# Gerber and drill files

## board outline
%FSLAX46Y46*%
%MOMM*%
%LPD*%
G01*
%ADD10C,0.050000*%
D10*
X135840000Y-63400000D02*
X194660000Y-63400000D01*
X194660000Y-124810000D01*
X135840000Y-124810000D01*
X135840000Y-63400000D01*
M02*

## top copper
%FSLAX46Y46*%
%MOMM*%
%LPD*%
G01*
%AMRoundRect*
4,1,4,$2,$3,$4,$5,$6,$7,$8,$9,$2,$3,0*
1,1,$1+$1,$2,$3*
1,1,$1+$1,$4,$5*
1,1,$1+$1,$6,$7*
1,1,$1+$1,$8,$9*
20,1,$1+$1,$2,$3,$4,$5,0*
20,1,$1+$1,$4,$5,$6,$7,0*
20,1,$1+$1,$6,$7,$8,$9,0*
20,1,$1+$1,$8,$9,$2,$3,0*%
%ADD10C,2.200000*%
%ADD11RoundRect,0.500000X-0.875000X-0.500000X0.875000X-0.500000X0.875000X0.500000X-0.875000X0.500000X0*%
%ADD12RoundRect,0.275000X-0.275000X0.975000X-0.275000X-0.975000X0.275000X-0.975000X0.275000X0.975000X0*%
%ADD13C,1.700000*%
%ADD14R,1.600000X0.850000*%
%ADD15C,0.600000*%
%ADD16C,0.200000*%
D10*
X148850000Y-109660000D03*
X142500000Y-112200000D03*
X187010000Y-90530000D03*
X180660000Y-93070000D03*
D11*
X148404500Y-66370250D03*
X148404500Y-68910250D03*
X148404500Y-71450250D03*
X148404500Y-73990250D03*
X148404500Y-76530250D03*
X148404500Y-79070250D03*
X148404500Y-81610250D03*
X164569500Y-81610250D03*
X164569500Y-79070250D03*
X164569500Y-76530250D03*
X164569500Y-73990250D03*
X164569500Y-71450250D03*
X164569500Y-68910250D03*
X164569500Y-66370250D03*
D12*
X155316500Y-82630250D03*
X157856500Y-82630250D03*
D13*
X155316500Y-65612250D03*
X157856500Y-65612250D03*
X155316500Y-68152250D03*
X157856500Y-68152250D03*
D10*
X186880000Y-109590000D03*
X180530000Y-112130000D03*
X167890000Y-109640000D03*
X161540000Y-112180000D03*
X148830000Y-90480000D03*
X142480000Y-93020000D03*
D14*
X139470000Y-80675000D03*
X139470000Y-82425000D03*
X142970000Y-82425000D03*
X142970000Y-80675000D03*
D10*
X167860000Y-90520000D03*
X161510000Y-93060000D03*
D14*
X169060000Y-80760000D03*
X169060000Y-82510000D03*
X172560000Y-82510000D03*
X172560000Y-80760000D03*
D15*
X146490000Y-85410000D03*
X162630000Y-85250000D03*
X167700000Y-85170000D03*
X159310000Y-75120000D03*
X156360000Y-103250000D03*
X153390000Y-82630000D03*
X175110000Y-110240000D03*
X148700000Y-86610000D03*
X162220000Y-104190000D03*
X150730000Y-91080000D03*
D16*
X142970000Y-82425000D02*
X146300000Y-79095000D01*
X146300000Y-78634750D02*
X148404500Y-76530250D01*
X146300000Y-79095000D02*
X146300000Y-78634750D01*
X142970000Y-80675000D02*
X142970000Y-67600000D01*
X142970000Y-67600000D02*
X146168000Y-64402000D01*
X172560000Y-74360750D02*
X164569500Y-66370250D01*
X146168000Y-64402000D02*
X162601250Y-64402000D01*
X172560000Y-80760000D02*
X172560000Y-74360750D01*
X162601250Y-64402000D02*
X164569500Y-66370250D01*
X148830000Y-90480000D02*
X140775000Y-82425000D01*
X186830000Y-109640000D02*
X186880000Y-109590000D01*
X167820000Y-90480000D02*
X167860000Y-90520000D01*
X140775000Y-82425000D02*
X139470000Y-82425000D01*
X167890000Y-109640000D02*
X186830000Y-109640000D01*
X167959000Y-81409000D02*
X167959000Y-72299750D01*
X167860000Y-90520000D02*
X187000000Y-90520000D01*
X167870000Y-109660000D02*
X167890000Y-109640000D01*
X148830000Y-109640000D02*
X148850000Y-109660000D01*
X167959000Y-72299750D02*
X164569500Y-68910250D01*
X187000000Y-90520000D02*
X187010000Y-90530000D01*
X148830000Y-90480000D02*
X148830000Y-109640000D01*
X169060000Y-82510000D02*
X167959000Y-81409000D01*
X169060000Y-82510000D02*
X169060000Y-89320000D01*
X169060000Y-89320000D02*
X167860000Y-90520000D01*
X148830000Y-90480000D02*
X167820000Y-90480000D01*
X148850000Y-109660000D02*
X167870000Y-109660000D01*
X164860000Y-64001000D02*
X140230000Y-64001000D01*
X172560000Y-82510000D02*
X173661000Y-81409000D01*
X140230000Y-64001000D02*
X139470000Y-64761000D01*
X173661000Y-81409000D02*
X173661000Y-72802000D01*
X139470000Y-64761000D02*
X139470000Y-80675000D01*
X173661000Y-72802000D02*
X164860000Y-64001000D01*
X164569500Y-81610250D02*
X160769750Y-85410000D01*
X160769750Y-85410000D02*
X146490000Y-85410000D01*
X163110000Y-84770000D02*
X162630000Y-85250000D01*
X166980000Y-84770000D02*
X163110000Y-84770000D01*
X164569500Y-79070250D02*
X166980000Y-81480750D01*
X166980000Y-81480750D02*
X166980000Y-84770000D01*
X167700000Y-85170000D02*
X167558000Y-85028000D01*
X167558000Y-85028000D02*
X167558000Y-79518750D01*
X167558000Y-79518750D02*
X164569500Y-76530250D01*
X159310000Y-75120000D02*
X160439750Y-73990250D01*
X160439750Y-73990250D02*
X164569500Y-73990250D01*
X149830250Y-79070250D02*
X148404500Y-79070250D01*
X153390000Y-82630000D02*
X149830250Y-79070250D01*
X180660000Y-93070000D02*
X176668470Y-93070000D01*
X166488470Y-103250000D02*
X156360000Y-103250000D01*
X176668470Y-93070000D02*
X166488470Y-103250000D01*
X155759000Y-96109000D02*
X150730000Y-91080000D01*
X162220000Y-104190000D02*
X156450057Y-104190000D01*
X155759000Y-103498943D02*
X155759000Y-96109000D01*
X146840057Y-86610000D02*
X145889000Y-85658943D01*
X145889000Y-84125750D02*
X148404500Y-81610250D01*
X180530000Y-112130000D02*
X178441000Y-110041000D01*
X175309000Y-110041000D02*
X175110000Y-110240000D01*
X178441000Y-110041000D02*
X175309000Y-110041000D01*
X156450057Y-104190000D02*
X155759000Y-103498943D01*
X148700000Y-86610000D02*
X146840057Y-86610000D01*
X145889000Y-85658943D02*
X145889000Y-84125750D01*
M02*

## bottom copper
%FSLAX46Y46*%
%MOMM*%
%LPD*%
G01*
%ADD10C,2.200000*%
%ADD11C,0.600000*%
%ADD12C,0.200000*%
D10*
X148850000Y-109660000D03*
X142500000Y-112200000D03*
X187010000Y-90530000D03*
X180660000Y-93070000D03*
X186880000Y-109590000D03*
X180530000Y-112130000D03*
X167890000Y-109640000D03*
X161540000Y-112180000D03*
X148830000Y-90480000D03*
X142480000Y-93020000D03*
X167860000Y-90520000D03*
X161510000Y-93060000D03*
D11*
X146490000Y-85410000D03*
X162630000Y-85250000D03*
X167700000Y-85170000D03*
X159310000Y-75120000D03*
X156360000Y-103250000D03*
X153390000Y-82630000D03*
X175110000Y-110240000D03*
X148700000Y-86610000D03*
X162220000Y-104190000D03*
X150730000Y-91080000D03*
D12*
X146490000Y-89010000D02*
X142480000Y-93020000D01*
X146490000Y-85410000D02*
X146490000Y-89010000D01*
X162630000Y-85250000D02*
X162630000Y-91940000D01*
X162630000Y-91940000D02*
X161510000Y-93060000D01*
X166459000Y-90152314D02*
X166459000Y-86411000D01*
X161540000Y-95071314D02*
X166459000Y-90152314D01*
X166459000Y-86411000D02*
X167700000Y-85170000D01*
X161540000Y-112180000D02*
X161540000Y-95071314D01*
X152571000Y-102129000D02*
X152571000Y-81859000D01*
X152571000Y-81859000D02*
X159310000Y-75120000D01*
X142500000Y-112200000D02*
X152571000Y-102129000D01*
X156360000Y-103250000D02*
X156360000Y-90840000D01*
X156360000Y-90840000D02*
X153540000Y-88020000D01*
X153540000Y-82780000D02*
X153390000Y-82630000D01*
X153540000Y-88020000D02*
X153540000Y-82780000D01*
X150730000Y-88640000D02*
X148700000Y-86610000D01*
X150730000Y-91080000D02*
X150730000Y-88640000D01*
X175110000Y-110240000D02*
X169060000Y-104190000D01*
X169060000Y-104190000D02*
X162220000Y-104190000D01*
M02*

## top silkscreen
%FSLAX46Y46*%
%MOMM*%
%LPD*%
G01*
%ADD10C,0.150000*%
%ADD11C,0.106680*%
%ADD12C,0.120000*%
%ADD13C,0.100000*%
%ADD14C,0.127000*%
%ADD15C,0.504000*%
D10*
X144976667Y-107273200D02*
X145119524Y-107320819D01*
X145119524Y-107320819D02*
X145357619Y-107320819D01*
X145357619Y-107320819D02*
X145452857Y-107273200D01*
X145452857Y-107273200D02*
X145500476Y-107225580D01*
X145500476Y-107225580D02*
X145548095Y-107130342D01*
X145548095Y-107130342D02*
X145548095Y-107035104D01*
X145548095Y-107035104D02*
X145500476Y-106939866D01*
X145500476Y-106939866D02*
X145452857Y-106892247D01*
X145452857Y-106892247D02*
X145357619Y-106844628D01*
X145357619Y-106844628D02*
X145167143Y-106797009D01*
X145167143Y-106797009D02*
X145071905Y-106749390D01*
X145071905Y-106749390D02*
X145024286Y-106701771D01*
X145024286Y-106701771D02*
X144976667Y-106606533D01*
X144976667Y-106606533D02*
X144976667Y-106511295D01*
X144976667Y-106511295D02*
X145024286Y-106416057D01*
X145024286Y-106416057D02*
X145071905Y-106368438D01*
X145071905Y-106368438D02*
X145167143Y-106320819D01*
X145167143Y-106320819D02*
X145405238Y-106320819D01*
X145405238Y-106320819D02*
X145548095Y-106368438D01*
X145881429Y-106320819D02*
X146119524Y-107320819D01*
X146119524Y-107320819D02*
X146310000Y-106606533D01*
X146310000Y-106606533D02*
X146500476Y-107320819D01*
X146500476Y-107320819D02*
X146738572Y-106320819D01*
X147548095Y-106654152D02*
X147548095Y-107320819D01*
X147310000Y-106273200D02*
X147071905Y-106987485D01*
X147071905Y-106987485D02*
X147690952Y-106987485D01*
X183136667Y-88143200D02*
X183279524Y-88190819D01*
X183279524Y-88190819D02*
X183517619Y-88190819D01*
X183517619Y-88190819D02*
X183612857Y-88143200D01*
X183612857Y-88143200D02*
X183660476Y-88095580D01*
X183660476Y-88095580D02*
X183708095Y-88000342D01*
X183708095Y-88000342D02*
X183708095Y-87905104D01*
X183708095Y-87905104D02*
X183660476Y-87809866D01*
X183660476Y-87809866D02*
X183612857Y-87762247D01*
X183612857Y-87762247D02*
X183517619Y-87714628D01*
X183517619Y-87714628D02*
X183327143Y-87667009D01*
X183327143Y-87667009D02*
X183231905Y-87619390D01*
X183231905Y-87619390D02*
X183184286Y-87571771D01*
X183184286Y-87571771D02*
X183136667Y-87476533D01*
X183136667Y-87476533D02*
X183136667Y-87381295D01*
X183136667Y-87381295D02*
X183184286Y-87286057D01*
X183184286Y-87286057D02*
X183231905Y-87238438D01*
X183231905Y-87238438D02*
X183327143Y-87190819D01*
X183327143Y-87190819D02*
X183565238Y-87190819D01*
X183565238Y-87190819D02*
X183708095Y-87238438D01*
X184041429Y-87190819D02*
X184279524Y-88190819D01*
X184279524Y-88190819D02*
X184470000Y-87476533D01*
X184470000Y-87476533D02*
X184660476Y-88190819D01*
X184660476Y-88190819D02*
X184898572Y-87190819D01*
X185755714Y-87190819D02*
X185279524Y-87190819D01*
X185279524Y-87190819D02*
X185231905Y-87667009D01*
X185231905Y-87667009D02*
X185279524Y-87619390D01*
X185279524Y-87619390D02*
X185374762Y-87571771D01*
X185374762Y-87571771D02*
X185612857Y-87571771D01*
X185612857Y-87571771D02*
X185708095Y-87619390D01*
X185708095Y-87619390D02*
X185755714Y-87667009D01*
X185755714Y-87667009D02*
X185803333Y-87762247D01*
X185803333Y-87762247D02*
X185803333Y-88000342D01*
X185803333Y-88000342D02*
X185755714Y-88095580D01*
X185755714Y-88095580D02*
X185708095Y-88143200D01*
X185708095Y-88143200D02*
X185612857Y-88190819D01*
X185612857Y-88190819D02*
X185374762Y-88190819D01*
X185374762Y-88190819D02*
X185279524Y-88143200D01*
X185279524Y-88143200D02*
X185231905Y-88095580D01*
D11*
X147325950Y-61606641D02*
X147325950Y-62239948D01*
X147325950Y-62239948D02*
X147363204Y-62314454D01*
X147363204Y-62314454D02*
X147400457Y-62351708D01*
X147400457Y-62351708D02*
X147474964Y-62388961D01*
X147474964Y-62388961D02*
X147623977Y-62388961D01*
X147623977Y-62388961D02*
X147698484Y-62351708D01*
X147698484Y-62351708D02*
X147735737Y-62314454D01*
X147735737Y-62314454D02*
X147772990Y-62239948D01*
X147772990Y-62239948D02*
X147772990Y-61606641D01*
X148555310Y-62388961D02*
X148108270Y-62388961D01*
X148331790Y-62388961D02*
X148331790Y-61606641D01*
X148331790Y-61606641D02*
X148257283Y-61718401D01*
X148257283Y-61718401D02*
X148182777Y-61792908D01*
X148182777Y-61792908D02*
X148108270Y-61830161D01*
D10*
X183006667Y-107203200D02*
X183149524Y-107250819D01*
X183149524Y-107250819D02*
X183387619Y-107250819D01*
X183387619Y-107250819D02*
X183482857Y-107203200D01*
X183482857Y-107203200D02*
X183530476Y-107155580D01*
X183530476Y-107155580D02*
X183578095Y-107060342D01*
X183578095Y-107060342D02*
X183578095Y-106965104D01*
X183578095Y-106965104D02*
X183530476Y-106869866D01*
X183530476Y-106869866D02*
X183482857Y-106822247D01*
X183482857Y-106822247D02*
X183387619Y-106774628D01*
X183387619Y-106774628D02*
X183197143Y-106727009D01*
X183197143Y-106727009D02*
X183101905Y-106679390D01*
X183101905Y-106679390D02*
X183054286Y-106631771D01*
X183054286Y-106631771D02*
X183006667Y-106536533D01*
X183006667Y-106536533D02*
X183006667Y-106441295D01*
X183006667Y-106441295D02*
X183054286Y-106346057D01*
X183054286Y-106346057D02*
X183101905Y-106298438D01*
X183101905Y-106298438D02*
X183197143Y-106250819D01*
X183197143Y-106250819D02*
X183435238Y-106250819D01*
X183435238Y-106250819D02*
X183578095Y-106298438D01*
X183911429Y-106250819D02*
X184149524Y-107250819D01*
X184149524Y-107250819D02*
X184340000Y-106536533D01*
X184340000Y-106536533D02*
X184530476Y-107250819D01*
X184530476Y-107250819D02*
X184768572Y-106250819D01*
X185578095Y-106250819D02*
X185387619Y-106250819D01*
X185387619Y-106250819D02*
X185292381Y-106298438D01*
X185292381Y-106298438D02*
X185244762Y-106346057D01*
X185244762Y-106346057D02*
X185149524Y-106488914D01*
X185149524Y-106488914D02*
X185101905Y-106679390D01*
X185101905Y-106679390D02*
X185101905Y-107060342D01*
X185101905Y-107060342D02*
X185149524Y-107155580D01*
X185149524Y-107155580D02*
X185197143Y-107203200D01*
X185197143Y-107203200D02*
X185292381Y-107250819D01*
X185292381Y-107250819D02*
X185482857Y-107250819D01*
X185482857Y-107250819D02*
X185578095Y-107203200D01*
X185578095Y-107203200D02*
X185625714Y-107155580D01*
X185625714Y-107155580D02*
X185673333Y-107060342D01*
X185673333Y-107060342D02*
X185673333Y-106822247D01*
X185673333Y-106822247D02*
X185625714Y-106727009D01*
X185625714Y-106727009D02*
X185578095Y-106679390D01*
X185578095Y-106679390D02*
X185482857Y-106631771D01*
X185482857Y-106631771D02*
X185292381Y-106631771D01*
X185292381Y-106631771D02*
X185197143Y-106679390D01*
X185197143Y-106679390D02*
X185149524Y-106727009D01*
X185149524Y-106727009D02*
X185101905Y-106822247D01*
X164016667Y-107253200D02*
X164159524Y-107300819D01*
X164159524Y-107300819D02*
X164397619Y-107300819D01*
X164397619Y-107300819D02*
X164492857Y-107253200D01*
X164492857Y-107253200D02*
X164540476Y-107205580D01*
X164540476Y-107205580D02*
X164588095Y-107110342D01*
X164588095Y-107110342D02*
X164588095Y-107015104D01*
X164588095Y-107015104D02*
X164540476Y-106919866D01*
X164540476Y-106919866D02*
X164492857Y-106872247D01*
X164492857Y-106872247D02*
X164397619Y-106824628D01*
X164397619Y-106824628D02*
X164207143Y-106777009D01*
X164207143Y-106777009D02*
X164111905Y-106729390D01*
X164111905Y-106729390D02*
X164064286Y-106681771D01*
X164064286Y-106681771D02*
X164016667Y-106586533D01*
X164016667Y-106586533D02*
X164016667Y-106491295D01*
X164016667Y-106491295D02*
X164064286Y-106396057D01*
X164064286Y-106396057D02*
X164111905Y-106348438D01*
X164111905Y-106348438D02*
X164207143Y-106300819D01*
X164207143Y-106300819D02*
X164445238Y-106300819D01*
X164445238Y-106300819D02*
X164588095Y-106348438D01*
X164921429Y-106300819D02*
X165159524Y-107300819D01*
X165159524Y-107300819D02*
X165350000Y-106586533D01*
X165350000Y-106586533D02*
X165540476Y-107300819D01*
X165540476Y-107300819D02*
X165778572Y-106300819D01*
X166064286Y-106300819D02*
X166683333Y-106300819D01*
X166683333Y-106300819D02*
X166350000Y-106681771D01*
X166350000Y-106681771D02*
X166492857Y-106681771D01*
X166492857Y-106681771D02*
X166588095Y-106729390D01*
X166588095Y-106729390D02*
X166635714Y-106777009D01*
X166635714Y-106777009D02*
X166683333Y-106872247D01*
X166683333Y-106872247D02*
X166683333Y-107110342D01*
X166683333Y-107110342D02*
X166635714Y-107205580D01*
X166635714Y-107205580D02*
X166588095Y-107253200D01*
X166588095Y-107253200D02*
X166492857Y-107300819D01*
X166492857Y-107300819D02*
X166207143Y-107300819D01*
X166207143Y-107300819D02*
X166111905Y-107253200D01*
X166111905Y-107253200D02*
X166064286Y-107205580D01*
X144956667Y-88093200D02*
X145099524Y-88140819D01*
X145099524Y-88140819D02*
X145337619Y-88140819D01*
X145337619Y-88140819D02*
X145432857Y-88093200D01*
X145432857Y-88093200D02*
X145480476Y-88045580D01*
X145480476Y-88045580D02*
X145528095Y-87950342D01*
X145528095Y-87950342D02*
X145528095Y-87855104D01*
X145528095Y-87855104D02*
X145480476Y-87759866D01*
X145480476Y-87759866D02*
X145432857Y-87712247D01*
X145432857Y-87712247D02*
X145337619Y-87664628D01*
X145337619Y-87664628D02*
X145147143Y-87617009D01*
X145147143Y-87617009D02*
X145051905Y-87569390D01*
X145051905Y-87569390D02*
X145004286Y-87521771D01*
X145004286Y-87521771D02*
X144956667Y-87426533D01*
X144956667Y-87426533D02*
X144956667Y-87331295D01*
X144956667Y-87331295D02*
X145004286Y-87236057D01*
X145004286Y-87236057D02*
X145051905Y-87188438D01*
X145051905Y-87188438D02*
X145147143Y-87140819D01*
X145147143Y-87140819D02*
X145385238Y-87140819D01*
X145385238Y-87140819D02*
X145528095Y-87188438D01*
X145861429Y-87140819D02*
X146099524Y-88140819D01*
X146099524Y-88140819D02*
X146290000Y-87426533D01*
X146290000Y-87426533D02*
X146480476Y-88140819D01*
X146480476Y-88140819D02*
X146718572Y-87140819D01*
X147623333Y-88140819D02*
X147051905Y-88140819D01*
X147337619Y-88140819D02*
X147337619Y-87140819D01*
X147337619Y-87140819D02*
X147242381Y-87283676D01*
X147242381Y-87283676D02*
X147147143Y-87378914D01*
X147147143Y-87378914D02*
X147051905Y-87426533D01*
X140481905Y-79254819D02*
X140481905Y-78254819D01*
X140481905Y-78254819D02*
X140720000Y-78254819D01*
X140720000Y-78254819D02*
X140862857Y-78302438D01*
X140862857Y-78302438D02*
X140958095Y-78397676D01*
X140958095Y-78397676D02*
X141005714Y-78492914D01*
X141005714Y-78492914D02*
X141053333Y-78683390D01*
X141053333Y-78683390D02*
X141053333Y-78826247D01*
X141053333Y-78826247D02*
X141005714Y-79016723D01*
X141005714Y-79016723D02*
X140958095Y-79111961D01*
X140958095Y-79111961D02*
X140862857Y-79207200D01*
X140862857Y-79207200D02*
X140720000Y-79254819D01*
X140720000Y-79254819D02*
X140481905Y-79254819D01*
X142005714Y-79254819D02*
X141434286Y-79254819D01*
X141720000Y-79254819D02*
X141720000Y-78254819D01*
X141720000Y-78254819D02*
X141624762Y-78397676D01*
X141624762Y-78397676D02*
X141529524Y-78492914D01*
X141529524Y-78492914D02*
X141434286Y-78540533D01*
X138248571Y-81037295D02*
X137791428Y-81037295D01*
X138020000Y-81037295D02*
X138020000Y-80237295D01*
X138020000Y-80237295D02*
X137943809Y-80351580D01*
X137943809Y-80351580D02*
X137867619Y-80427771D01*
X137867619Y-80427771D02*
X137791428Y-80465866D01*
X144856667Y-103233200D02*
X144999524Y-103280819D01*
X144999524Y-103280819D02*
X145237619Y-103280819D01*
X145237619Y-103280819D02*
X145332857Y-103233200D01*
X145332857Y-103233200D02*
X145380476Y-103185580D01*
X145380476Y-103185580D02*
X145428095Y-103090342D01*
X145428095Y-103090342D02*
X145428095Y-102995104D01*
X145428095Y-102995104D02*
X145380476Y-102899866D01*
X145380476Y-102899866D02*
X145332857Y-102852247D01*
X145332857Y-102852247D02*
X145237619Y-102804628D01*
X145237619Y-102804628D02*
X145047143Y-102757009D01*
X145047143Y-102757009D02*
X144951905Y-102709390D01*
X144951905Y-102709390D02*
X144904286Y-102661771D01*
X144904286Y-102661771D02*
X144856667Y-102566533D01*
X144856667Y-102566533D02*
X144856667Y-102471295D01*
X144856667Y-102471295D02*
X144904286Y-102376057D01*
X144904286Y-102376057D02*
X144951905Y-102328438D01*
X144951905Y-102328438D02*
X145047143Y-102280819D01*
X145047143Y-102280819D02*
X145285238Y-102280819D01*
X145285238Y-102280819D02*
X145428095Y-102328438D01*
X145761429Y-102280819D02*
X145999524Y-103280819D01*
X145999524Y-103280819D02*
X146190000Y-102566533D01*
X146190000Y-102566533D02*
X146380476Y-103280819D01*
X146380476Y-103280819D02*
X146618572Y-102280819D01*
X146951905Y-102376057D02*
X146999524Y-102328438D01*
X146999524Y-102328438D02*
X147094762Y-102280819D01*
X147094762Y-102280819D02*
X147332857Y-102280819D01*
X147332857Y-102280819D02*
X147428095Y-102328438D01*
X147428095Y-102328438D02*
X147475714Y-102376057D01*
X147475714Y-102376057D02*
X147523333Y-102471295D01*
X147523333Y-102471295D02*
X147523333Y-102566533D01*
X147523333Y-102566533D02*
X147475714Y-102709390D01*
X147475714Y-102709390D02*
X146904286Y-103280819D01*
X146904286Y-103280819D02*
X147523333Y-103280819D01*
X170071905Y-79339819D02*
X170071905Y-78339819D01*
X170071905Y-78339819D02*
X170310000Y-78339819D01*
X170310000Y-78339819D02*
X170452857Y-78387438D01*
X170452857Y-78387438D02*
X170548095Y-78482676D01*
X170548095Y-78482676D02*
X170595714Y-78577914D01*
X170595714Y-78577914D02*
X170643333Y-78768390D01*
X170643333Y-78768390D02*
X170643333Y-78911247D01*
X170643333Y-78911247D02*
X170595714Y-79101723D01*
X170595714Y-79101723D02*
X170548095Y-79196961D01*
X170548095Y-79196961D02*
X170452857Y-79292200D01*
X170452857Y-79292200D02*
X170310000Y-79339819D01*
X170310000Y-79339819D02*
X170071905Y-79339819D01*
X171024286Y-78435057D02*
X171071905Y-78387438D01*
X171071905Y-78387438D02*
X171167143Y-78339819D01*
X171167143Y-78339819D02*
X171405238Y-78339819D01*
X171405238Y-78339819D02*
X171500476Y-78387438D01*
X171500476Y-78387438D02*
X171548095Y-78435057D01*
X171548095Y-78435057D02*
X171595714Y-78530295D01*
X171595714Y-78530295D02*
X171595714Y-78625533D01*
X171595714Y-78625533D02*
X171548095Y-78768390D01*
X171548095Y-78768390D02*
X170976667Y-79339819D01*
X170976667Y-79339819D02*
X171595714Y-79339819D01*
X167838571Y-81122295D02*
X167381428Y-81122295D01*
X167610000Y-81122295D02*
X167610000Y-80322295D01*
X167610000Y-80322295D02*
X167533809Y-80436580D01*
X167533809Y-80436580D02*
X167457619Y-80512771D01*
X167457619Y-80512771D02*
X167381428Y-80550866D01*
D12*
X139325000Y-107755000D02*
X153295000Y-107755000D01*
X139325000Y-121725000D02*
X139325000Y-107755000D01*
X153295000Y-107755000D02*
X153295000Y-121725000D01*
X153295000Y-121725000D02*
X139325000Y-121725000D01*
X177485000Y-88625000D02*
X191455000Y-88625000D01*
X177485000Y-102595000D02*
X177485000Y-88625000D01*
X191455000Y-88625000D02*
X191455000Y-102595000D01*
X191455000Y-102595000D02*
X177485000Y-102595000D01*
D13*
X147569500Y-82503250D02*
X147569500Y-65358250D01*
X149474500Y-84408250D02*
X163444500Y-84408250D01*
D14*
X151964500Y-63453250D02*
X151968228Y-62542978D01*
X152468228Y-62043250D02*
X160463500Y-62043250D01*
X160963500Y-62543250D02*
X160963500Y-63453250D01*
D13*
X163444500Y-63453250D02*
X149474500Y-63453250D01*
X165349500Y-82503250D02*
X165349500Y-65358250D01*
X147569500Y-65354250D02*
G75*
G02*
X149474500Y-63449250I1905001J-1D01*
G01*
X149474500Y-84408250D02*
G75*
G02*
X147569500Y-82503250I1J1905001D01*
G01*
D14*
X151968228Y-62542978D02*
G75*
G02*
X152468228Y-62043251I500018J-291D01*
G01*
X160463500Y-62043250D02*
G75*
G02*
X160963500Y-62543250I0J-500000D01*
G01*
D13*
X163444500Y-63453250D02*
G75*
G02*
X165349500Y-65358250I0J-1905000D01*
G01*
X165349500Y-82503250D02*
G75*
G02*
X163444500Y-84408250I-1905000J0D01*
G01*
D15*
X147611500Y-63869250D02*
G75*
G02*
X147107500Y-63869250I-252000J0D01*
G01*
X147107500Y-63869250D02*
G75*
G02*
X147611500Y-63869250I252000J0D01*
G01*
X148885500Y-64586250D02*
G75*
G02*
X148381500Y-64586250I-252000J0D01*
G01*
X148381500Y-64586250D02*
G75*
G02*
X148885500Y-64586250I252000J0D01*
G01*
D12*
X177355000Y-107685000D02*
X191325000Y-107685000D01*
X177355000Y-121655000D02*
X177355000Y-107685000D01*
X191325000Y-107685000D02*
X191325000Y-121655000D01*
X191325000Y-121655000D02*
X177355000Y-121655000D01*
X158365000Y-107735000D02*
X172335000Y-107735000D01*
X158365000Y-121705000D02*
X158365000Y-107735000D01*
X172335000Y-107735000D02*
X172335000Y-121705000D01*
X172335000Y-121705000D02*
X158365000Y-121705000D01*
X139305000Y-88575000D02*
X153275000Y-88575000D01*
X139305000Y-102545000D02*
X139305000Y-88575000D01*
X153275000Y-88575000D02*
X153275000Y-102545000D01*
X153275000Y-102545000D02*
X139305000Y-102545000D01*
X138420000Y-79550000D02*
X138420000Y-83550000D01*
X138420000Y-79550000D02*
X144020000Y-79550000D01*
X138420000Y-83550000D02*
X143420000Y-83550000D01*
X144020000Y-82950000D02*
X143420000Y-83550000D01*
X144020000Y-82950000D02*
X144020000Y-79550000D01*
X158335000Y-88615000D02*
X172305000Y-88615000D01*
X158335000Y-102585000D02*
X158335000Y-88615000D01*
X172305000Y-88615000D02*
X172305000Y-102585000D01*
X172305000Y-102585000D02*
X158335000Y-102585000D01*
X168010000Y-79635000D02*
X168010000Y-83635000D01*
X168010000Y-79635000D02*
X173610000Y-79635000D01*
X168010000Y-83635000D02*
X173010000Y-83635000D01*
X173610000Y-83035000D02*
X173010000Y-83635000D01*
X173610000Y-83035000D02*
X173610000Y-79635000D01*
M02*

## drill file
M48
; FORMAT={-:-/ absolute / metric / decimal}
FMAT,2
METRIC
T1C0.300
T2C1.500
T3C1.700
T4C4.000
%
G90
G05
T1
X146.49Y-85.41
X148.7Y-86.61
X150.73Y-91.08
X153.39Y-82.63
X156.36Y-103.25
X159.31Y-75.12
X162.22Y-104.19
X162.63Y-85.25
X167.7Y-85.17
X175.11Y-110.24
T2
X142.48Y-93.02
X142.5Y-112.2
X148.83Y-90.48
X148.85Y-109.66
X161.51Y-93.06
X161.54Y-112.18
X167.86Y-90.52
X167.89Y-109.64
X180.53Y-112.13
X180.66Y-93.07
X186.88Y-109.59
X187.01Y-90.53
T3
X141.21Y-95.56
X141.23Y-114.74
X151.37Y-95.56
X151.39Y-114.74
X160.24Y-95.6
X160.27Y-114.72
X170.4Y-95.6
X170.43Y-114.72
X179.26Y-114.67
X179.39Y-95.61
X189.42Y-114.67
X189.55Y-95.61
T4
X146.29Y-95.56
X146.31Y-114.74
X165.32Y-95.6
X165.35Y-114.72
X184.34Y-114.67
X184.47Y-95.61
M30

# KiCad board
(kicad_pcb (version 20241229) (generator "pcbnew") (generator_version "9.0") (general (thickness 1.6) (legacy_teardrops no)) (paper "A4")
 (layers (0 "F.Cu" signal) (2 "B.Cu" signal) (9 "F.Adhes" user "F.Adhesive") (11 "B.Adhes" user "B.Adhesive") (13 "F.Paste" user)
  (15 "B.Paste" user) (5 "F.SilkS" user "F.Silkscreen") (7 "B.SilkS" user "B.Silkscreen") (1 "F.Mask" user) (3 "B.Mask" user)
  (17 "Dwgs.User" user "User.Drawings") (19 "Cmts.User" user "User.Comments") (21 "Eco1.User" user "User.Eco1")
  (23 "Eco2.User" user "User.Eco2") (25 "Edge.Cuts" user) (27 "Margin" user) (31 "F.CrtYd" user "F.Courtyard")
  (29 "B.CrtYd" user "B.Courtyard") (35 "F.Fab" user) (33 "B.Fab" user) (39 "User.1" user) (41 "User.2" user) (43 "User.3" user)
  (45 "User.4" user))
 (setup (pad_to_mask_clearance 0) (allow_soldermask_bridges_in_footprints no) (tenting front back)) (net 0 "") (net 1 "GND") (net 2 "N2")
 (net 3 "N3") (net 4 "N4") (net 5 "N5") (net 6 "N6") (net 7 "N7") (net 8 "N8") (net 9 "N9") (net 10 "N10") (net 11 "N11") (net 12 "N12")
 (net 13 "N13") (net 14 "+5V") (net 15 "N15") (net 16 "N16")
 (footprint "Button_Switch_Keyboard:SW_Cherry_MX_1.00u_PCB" (layer "F.Cu") (at 148.85 109.66)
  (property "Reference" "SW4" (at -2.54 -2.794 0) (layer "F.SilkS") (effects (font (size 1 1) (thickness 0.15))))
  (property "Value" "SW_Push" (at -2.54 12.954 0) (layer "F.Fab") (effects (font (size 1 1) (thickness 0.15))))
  (fp_line (start -9.525 -1.905) (end 4.445 -1.905) (stroke (width 0.12) (type solid)) (layer "F.SilkS"))
  (fp_line (start -9.525 12.065) (end -9.525 -1.905) (stroke (width 0.12) (type solid)) (layer "F.SilkS"))
  (fp_line (start 4.445 -1.905) (end 4.445 12.065) (stroke (width 0.12) (type solid)) (layer "F.SilkS"))
  (fp_line (start 4.445 12.065) (end -9.525 12.065) (stroke (width 0.12) (type solid)) (layer "F.SilkS"))
  (pad "" np_thru_hole circle (at -7.62 5.08) (size 1.7 1.7) (drill 1.7) (layers "*.Cu" "*.Mask"))
  (pad "" np_thru_hole circle (at -2.54 5.08) (size 4 4) (drill 4) (layers "*.Cu" "*.Mask"))
  (pad "" np_thru_hole circle (at 2.54 5.08) (size 1.7 1.7) (drill 1.7) (layers "*.Cu" "*.Mask"))
  (pad "1" thru_hole circle (at 0 0) (size 2.2 2.2) (drill 1.5) (layers "*.Cu" "*.Mask") (remove_unused_layers no) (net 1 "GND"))
  (pad "2" thru_hole circle (at -6.35 2.54) (size 2.2 2.2) (drill 1.5) (layers "*.Cu" "*.Mask") (remove_unused_layers no) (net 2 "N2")))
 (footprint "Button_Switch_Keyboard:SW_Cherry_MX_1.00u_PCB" (layer "F.Cu") (at 187.01 90.53)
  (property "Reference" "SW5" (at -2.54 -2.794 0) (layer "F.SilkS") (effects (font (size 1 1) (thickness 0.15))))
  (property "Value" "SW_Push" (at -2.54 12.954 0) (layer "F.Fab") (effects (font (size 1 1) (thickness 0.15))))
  (fp_line (start -9.525 -1.905) (end 4.445 -1.905) (stroke (width 0.12) (type solid)) (layer "F.SilkS"))
  (fp_line (start -9.525 12.065) (end -9.525 -1.905) (stroke (width 0.12) (type solid)) (layer "F.SilkS"))
  (fp_line (start 4.445 -1.905) (end 4.445 12.065) (stroke (width 0.12) (type solid)) (layer "F.SilkS"))
  (fp_line (start 4.445 12.065) (end -9.525 12.065) (stroke (width 0.12) (type solid)) (layer "F.SilkS"))
  (pad "" np_thru_hole circle (at -7.62 5.08) (size 1.7 1.7) (drill 1.7) (layers "*.Cu" "*.Mask"))
  (pad "" np_thru_hole circle (at -2.54 5.08) (size 4 4) (drill 4) (layers "*.Cu" "*.Mask"))
  (pad "" np_thru_hole circle (at 2.54 5.08) (size 1.7 1.7) (drill 1.7) (layers "*.Cu" "*.Mask"))
  (pad "1" thru_hole circle (at 0 0) (size 2.2 2.2) (drill 1.5) (layers "*.Cu" "*.Mask") (remove_unused_layers no) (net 1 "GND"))
  (pad "2" thru_hole circle (at -6.35 2.54) (size 2.2 2.2) (drill 1.5) (layers "*.Cu" "*.Mask") (remove_unused_layers no) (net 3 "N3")))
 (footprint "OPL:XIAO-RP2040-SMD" (layer "F.Cu") (at 156.4045 73.99025)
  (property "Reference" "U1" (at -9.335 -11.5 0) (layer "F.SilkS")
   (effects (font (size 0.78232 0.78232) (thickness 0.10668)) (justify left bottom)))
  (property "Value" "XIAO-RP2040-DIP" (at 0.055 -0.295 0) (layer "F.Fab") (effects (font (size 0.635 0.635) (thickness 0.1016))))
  (fp_line (start -8.835 8.513) (end -8.835 -8.632) (stroke (width 0.1) (type solid)) (layer "F.SilkS"))
  (fp_line (start -6.93 10.418) (end 7.04 10.418) (stroke (width 0.1) (type solid)) (layer "F.SilkS"))
  (fp_line (start -4.44 -10.537) (end -4.436272 -11.447272) (stroke (width 0.127) (type solid)) (layer "F.SilkS"))
  (fp_line (start -3.936272 -11.947) (end 4.059 -11.947) (stroke (width 0.127) (type solid)) (layer "F.SilkS"))
  (fp_line (start 4.559 -11.447) (end 4.559 -10.537) (stroke (width 0.127) (type solid)) (layer "F.SilkS"))
  (fp_line (start 7.04 -10.537) (end -6.93 -10.537) (stroke (width 0.1) (type solid)) (layer "F.SilkS"))
  (fp_line (start 8.945 8.513) (end 8.945 -8.632) (stroke (width 0.1) (type solid)) (layer "F.SilkS"))
  (fp_arc (start -8.835 -8.636) (mid -8.277038 -9.983038) (end -6.93 -10.541) (stroke (width 0.1) (type solid)) (layer "F.SilkS"))
  (fp_arc (start -6.93 10.418) (mid -8.277038 9.860038) (end -8.835 8.513) (stroke (width 0.1) (type solid)) (layer "F.SilkS"))
  (fp_arc (start -4.436272 -11.447272) (mid -4.289724 -11.800644) (end -3.936272 -11.947) (stroke (width 0.127) (type default))
   (layer "F.SilkS"))
  (fp_arc (start 4.059 -11.947) (mid 4.412553 -11.800553) (end 4.559 -11.447) (stroke (width 0.127) (type default)) (layer "F.SilkS"))
  (fp_arc (start 7.04 -10.537) (mid 8.387038 -9.979038) (end 8.945 -8.632) (stroke (width 0.1) (type solid)) (layer "F.SilkS"))
  (fp_arc (start 8.945 8.513) (mid 8.387038 9.860038) (end 7.04 10.418) (stroke (width 0.1) (type solid)) (layer "F.SilkS"))
  (fp_circle (center -9.045 -10.121) (end -9.045 -10.375) (stroke (width 0.5) (type solid)) (fill yes) (layer "F.SilkS"))
  (fp_circle (center -7.771 -9.404) (end -7.771 -9.658) (stroke (width 0.5) (type solid)) (fill yes) (layer "F.SilkS"))
  (pad "1" smd roundrect (at -8 -7.62) (size 2.75 2) (layers "F.Cu" "F.Mask" "F.Paste") (roundrect_rratio 0.25) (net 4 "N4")
   (solder_mask_margin 0.0508) (thermal_bridge_angle 45))
  (pad "2" smd roundrect (at -8 -5.08) (size 2.75 2) (layers "F.Cu" "F.Mask" "F.Paste") (roundrect_rratio 0.25) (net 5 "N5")
   (solder_mask_margin 0.0508) (thermal_bridge_angle 45))
  (pad "3" smd roundrect (at -8 -2.54) (size 2.75 2) (layers "F.Cu" "F.Mask" "F.Paste") (roundrect_rratio 0.25) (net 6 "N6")
   (solder_mask_margin 0.0508) (thermal_bridge_angle 45))
  (pad "4" smd roundrect (at -8 0) (size 2.75 2) (layers "F.Cu" "F.Mask" "F.Paste") (roundrect_rratio 0.25) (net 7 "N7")
   (solder_mask_margin 0.0508) (thermal_bridge_angle 45))
  (pad "5" smd roundrect (at -8 2.54) (size 2.75 2) (layers "F.Cu" "F.Mask" "F.Paste") (roundrect_rratio 0.25) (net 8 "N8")
   (solder_mask_margin 0.0508) (thermal_bridge_angle 45))
  (pad "6" smd roundrect (at -8 5.08) (size 2.75 2) (layers "F.Cu" "F.Mask" "F.Paste") (roundrect_rratio 0.25) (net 3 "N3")
   (solder_mask_margin 0.0508) (thermal_bridge_angle 45))
  (pad "7" smd roundrect (at -8 7.62) (size 2.75 2) (layers "F.Cu" "F.Mask" "F.Paste") (roundrect_rratio 0.25) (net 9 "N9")
   (solder_mask_margin 0.0508) (thermal_bridge_angle 45))
  (pad "8" smd roundrect (at 8.165 7.62) (size 2.75 2) (layers "F.Cu" "F.Mask" "F.Paste") (roundrect_rratio 0.25) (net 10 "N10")
   (solder_mask_margin 0.0508) (thermal_bridge_angle 45))
  (pad "9" smd roundrect (at 8.165 5.08) (size 2.75 2) (layers "F.Cu" "F.Mask" "F.Paste") (roundrect_rratio 0.25) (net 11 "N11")
   (solder_mask_margin 0.0508) (thermal_bridge_angle 45))
  (pad "10" smd roundrect (at 8.165 2.54) (size 2.75 2) (layers "F.Cu" "F.Mask" "F.Paste") (roundrect_rratio 0.25) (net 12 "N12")
   (solder_mask_margin 0.0508) (thermal_bridge_angle 45))
  (pad "11" smd roundrect (at 8.165 0) (size 2.75 2) (layers "F.Cu" "F.Mask" "F.Paste") (roundrect_rratio 0.25) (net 2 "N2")
   (solder_mask_margin 0.0508) (thermal_bridge_angle 45))
  (pad "12" smd roundrect (at 8.165 -2.54) (size 2.75 2) (layers "F.Cu" "F.Mask" "F.Paste") (roundrect_rratio 0.25) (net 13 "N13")
   (solder_mask_margin 0.0508) (thermal_bridge_angle 45))
  (pad "13" smd roundrect (at 8.165 -5.08) (size 2.75 2) (layers "F.Cu" "F.Mask" "F.Paste") (roundrect_rratio 0.25) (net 1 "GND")
   (solder_mask_margin 0.0508) (thermal_bridge_angle 45))
  (pad "14" smd roundrect (at 8.165 -7.62) (size 2.75 2) (layers "F.Cu" "F.Mask" "F.Paste") (roundrect_rratio 0.25) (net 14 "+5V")
   (solder_mask_margin 0.0508) (thermal_bridge_angle 45))
  (pad "15" smd roundrect (at -1.088 8.64 270) (size 2.5 1.1) (layers "F.Cu" "F.Mask" "F.Paste") (roundrect_rratio 0.25)
   (thermal_bridge_angle 45))
  (pad "16" smd roundrect (at 1.452 8.64 270) (size 2.5 1.1) (layers "F.Cu" "F.Mask" "F.Paste") (roundrect_rratio 0.25)
   (thermal_bridge_angle 45))
  (pad "17" smd circle (at -1.088 -8.378) (size 1.7 1.7) (layers "F.Cu" "F.Mask" "F.Paste"))
  (pad "18" smd circle (at 1.452 -8.378) (size 1.7 1.7) (layers "F.Cu" "F.Mask" "F.Paste"))
  (pad "19" smd circle (at -1.088 -5.838) (size 1.7 1.7) (layers "F.Cu" "F.Mask" "F.Paste"))
  (pad "20" smd circle (at 1.452 -5.838) (size 1.7 1.7) (layers "F.Cu" "F.Mask" "F.Paste")))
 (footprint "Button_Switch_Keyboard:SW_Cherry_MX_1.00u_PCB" (layer "F.Cu") (at 186.88 109.59)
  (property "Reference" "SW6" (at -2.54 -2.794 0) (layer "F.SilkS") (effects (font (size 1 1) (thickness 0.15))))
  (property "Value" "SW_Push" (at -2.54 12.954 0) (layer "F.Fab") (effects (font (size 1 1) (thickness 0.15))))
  (fp_line (start -9.525 -1.905) (end 4.445 -1.905) (stroke (width 0.12) (type solid)) (layer "F.SilkS"))
  (fp_line (start -9.525 12.065) (end -9.525 -1.905) (stroke (width 0.12) (type solid)) (layer "F.SilkS"))
  (fp_line (start 4.445 -1.905) (end 4.445 12.065) (stroke (width 0.12) (type solid)) (layer "F.SilkS"))
  (fp_line (start 4.445 12.065) (end -9.525 12.065) (stroke (width 0.12) (type solid)) (layer "F.SilkS"))
  (pad "" np_thru_hole circle (at -7.62 5.08) (size 1.7 1.7) (drill 1.7) (layers "*.Cu" "*.Mask"))
  (pad "" np_thru_hole circle (at -2.54 5.08) (size 4 4) (drill 4) (layers "*.Cu" "*.Mask"))
  (pad "" np_thru_hole circle (at 2.54 5.08) (size 1.7 1.7) (drill 1.7) (layers "*.Cu" "*.Mask"))
  (pad "1" thru_hole circle (at 0 0) (size 2.2 2.2) (drill 1.5) (layers "*.Cu" "*.Mask") (remove_unused_layers no) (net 1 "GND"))
  (pad "2" thru_hole circle (at -6.35 2.54) (size 2.2 2.2) (drill 1.5) (layers "*.Cu" "*.Mask") (remove_unused_layers no) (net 9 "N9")))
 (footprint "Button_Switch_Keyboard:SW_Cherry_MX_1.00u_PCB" (layer "F.Cu") (at 167.89 109.64)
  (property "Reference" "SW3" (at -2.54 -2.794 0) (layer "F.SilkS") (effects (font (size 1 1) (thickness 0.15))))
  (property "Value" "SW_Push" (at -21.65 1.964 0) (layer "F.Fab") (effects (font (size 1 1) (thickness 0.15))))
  (fp_line (start -9.525 -1.905) (end 4.445 -1.905) (stroke (width 0.12) (type solid)) (layer "F.SilkS"))
  (fp_line (start -9.525 12.065) (end -9.525 -1.905) (stroke (width 0.12) (type solid)) (layer "F.SilkS"))
  (fp_line (start 4.445 -1.905) (end 4.445 12.065) (stroke (width 0.12) (type solid)) (layer "F.SilkS"))
  (fp_line (start 4.445 12.065) (end -9.525 12.065) (stroke (width 0.12) (type solid)) (layer "F.SilkS"))
  (pad "" np_thru_hole circle (at -7.62 5.08) (size 1.7 1.7) (drill 1.7) (layers "*.Cu" "*.Mask"))
  (pad "" np_thru_hole circle (at -2.54 5.08) (size 4 4) (drill 4) (layers "*.Cu" "*.Mask"))
  (pad "" np_thru_hole circle (at 2.54 5.08) (size 1.7 1.7) (drill 1.7) (layers "*.Cu" "*.Mask"))
  (pad "1" thru_hole circle (at 0 0) (size 2.2 2.2) (drill 1.5) (layers "*.Cu" "*.Mask") (remove_unused_layers no) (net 1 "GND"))
  (pad "2" thru_hole circle (at -6.35 2.54) (size 2.2 2.2) (drill 1.5) (layers "*.Cu" "*.Mask") (remove_unused_layers no) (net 12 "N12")))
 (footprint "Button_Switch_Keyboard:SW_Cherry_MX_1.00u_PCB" (layer "F.Cu") (at 148.83 90.48)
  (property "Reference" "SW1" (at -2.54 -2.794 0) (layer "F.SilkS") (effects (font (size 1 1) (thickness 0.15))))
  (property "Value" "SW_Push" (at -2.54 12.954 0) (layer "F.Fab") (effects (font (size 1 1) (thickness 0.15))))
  (fp_line (start -9.525 -1.905) (end 4.445 -1.905) (stroke (width 0.12) (type solid)) (layer "F.SilkS"))
  (fp_line (start -9.525 12.065) (end -9.525 -1.905) (stroke (width 0.12) (type solid)) (layer "F.SilkS"))
  (fp_line (start 4.445 -1.905) (end 4.445 12.065) (stroke (width 0.12) (type solid)) (layer "F.SilkS"))
  (fp_line (start 4.445 12.065) (end -9.525 12.065) (stroke (width 0.12) (type solid)) (layer "F.SilkS"))
  (pad "" np_thru_hole circle (at -7.62 5.08) (size 1.7 1.7) (drill 1.7) (layers "*.Cu" "*.Mask"))
  (pad "" np_thru_hole circle (at -2.54 5.08) (size 4 4) (drill 4) (layers "*.Cu" "*.Mask"))
  (pad "" np_thru_hole circle (at 2.54 5.08) (size 1.7 1.7) (drill 1.7) (layers "*.Cu" "*.Mask"))
  (pad "1" thru_hole circle (at 0 0) (size 2.2 2.2) (drill 1.5) (layers "*.Cu" "*.Mask") (remove_unused_layers no) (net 1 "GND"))
  (pad "2" thru_hole circle (at -6.35 2.54) (size 2.2 2.2) (drill 1.5) (layers "*.Cu" "*.Mask") (remove_unused_layers no) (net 10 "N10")))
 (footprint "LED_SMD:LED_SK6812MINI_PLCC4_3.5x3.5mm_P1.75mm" (layer "F.Cu") (at 141.22 81.55)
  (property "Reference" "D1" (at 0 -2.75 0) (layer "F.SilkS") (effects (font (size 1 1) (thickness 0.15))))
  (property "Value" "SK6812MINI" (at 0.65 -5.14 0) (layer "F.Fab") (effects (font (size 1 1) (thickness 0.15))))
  (fp_line (start -2.8 -2) (end -2.8 2) (stroke (width 0.12) (type default)) (layer "F.SilkS"))
  (fp_line (start -2.8 -2) (end 2.8 -2) (stroke (width 0.12) (type solid)) (layer "F.SilkS"))
  (fp_line (start -2.8 2) (end 2.2 2) (stroke (width 0.12) (type solid)) (layer "F.SilkS"))
  (fp_line (start 2.8 1.4) (end 2.2 2) (stroke (width 0.12) (type default)) (layer "F.SilkS"))
  (fp_line (start 2.8 1.4) (end 2.8 -2) (stroke (width 0.12) (type solid)) (layer "F.SilkS"))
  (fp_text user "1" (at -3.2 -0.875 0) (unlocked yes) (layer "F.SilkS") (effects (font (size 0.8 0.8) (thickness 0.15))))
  (pad "1" smd rect (at -1.75 -0.875) (size 1.6 0.85) (layers "F.Cu" "F.Mask" "F.Paste") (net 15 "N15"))
  (pad "2" smd rect (at -1.75 0.875) (size 1.6 0.85) (layers "F.Cu" "F.Mask" "F.Paste") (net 1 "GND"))
  (pad "3" smd rect (at 1.75 0.875) (size 1.6 0.85) (layers "F.Cu" "F.Mask" "F.Paste") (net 8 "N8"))
  (pad "4" smd rect (at 1.75 -0.875) (size 1.6 0.85) (layers "F.Cu" "F.Mask" "F.Paste") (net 14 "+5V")))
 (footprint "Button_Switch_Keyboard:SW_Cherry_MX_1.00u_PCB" (layer "F.Cu") (at 167.86 90.52)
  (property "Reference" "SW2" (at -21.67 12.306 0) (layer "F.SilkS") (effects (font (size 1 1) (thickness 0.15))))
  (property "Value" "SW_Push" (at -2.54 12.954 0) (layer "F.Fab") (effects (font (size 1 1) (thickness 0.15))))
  (fp_line (start -9.525 -1.905) (end 4.445 -1.905) (stroke (width 0.12) (type solid)) (layer "F.SilkS"))
  (fp_line (start -9.525 12.065) (end -9.525 -1.905) (stroke (width 0.12) (type solid)) (layer "F.SilkS"))
  (fp_line (start 4.445 -1.905) (end 4.445 12.065) (stroke (width 0.12) (type solid)) (layer "F.SilkS"))
  (fp_line (start 4.445 12.065) (end -9.525 12.065) (stroke (width 0.12) (type solid)) (layer "F.SilkS"))
  (pad "" np_thru_hole circle (at -7.62 5.08) (size 1.7 1.7) (drill 1.7) (layers "*.Cu" "*.Mask"))
  (pad "" np_thru_hole circle (at -2.54 5.08) (size 4 4) (drill 4) (layers "*.Cu" "*.Mask"))
  (pad "" np_thru_hole circle (at 2.54 5.08) (size 1.7 1.7) (drill 1.7) (layers "*.Cu" "*.Mask"))
  (pad "1" thru_hole circle (at 0 0) (size 2.2 2.2) (drill 1.5) (layers "*.Cu" "*.Mask") (remove_unused_layers no) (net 1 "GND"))
  (pad "2" thru_hole circle (at -6.35 2.54) (size 2.2 2.2) (drill 1.5) (layers "*.Cu" "*.Mask") (remove_unused_layers no) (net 11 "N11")))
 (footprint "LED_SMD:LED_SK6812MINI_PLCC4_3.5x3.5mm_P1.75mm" (layer "F.Cu") (at 170.81 81.635)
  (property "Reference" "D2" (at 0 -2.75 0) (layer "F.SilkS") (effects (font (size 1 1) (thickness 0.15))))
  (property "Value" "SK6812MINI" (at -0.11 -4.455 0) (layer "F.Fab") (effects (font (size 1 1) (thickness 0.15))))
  (fp_line (start -2.8 -2) (end -2.8 2) (stroke (width 0.12) (type default)) (layer "F.SilkS"))
  (fp_line (start -2.8 -2) (end 2.8 -2) (stroke (width 0.12) (type solid)) (layer "F.SilkS"))
  (fp_line (start -2.8 2) (end 2.2 2) (stroke (width 0.12) (type solid)) (layer "F.SilkS"))
  (fp_line (start 2.8 1.4) (end 2.2 2) (stroke (width 0.12) (type default)) (layer "F.SilkS"))
  (fp_line (start 2.8 1.4) (end 2.8 -2) (stroke (width 0.12) (type solid)) (layer "F.SilkS"))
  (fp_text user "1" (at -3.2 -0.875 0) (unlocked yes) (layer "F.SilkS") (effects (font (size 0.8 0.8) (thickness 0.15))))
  (pad "1" smd rect (at -1.75 -0.875) (size 1.6 0.85) (layers "F.Cu" "F.Mask" "F.Paste") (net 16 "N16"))
  (pad "2" smd rect (at -1.75 0.875) (size 1.6 0.85) (layers "F.Cu" "F.Mask" "F.Paste") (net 1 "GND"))
  (pad "3" smd rect (at 1.75 0.875) (size 1.6 0.85) (layers "F.Cu" "F.Mask" "F.Paste") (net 15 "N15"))
  (pad "4" smd rect (at 1.75 -0.875) (size 1.6 0.85) (layers "F.Cu" "F.Mask" "F.Paste") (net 14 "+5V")))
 (gr_rect (start 135.84 63.4) (end 194.66 124.81) (stroke (width 0.05) (type default)) (fill no) (layer "Edge.Cuts"))
 (segment (start 142.97 82.425) (end 146.3 79.095) (width 0.2) (layer "F.Cu") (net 8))
 (segment (start 146.3 78.63475) (end 148.4045 76.53025) (width 0.2) (layer "F.Cu") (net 8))
 (segment (start 146.3 79.095) (end 146.3 78.63475) (width 0.2) (layer "F.Cu") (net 8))
 (segment (start 142.97 80.675) (end 142.97 67.6) (width 0.2) (layer "F.Cu") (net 14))
 (segment (start 142.97 67.6) (end 146.168 64.402) (width 0.2) (layer "F.Cu") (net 14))
 (segment (start 172.56 74.36075) (end 164.5695 66.37025) (width 0.2) (layer "F.Cu") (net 14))
 (segment (start 146.168 64.402) (end 162.60125 64.402) (width 0.2) (layer "F.Cu") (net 14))
 (segment (start 172.56 80.76) (end 172.56 74.36075) (width 0.2) (layer "F.Cu") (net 14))
 (segment (start 162.60125 64.402) (end 164.5695 66.37025) (width 0.2) (layer "F.Cu") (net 14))
 (segment (start 148.83 90.48) (end 140.775 82.425) (width 0.2) (layer "F.Cu") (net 1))
 (segment (start 186.83 109.64) (end 186.88 109.59) (width 0.2) (layer "F.Cu") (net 1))
 (segment (start 167.82 90.48) (end 167.86 90.52) (width 0.2) (layer "F.Cu") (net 1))
 (segment (start 140.775 82.425) (end 139.47 82.425) (width 0.2) (layer "F.Cu") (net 1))
 (segment (start 167.89 109.64) (end 186.83 109.64) (width 0.2) (layer "F.Cu") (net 1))
 (segment (start 167.959 81.409) (end 167.959 72.29975) (width 0.2) (layer "F.Cu") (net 1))
 (segment (start 167.86 90.52) (end 187 90.52) (width 0.2) (layer "F.Cu") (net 1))
 (segment (start 167.87 109.66) (end 167.89 109.64) (width 0.2) (layer "F.Cu") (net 1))
 (segment (start 148.83 109.64) (end 148.85 109.66) (width 0.2) (layer "F.Cu") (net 1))
 (segment (start 167.959 72.29975) (end 164.5695 68.91025) (width 0.2) (layer "F.Cu") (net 1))
 (segment (start 187 90.52) (end 187.01 90.53) (width 0.2) (layer "F.Cu") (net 1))
 (segment (start 148.83 90.48) (end 148.83 109.64) (width 0.2) (layer "F.Cu") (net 1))
 (segment (start 169.06 82.51) (end 167.959 81.409) (width 0.2) (layer "F.Cu") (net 1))
 (segment (start 169.06 82.51) (end 169.06 89.32) (width 0.2) (layer "F.Cu") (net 1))
 (segment (start 169.06 89.32) (end 167.86 90.52) (width 0.2) (layer "F.Cu") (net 1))
 (segment (start 148.83 90.48) (end 167.82 90.48) (width 0.2) (layer "F.Cu") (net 1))
 (segment (start 148.85 109.66) (end 167.87 109.66) (width 0.2) (layer "F.Cu") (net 1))
 (segment (start 164.86 64.001) (end 140.23 64.001) (width 0.2) (layer "F.Cu") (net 15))
 (segment (start 172.56 82.51) (end 173.661 81.409) (width 0.2) (layer "F.Cu") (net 15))
 (segment (start 140.23 64.001) (end 139.47 64.761) (width 0.2) (layer "F.Cu") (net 15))
 (segment (start 173.661 81.409) (end 173.661 72.802) (width 0.2) (layer "F.Cu") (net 15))
 (segment (start 139.47 64.761) (end 139.47 80.675) (width 0.2) (layer "F.Cu") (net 15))
 (segment (start 173.661 72.802) (end 164.86 64.001) (width 0.2) (layer "F.Cu") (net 15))
 (segment (start 164.5695 81.61025) (end 160.76975 85.41) (width 0.2) (layer "F.Cu") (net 10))
 (segment (start 160.76975 85.41) (end 146.49 85.41) (width 0.2) (layer "F.Cu") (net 10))
 (via (at 146.49 85.41) (size 0.6) (drill 0.3) (layers "F.Cu" "B.Cu") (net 10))
 (segment (start 146.49 89.01) (end 142.48 93.02) (width 0.2) (layer "B.Cu") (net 10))
 (segment (start 146.49 85.41) (end 146.49 89.01) (width 0.2) (layer "B.Cu") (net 10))
 (segment (start 163.11 84.77) (end 162.63 85.25) (width 0.2) (layer "F.Cu") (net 11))
 (segment (start 166.98 84.77) (end 163.11 84.77) (width 0.2) (layer "F.Cu") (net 11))
 (segment (start 164.5695 79.07025) (end 166.98 81.48075) (width 0.2) (layer "F.Cu") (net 11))
 (segment (start 166.98 81.48075) (end 166.98 84.77) (width 0.2) (layer "F.Cu") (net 11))
 (via (at 162.63 85.25) (size 0.6) (drill 0.3) (layers "F.Cu" "B.Cu") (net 11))
 (segment (start 162.63 85.25) (end 162.63 91.94) (width 0.2) (layer "B.Cu") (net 11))
 (segment (start 162.63 91.94) (end 161.51 93.06) (width 0.2) (layer "B.Cu") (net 11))
 (segment (start 167.7 85.17) (end 167.558 85.028) (width 0.2) (layer "F.Cu") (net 12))
 (segment (start 167.558 85.028) (end 167.558 79.51875) (width 0.2) (layer "F.Cu") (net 12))
 (segment (start 167.558 79.51875) (end 164.5695 76.53025) (width 0.2) (layer "F.Cu") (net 12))
 (via (at 167.7 85.17) (size 0.6) (drill 0.3) (layers "F.Cu" "B.Cu") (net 12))
 (segment (start 166.459 90.152314) (end 166.459 86.411) (width 0.2) (layer "B.Cu") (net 12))
 (segment (start 161.54 95.071314) (end 166.459 90.152314) (width 0.2) (layer "B.Cu") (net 12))
 (segment (start 166.459 86.411) (end 167.7 85.17) (width 0.2) (layer "B.Cu") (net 12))
 (segment (start 161.54 112.18) (end 161.54 95.071314) (width 0.2) (layer "B.Cu") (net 12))
 (segment (start 159.31 75.12) (end 160.43975 73.99025) (width 0.2) (layer "F.Cu") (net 2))
 (segment (start 160.43975 73.99025) (end 164.5695 73.99025) (width 0.2) (layer "F.Cu") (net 2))
 (via (at 159.31 75.12) (size 0.6) (drill 0.3) (layers "F.Cu" "B.Cu") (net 2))
 (segment (start 152.571 102.129) (end 152.571 81.859) (width 0.2) (layer "B.Cu") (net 2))
 (segment (start 152.571 81.859) (end 159.31 75.12) (width 0.2) (layer "B.Cu") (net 2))
 (segment (start 142.5 112.2) (end 152.571 102.129) (width 0.2) (layer "B.Cu") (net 2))
 (segment (start 149.83025 79.07025) (end 148.4045 79.07025) (width 0.2) (layer "F.Cu") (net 3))
 (segment (start 153.39 82.63) (end 149.83025 79.07025) (width 0.2) (layer "F.Cu") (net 3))
 (segment (start 180.66 93.07) (end 176.66847 93.07) (width 0.2) (layer "F.Cu") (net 3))
 (segment (start 166.48847 103.25) (end 156.36 103.25) (width 0.2) (layer "F.Cu") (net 3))
 (segment (start 176.66847 93.07) (end 166.48847 103.25) (width 0.2) (layer "F.Cu") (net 3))
 (via (at 156.36 103.25) (size 0.6) (drill 0.3) (layers "F.Cu" "B.Cu") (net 3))
 (via (at 153.39 82.63) (size 0.6) (drill 0.3) (layers "F.Cu" "B.Cu") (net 3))
 (segment (start 156.36 103.25) (end 156.36 90.84) (width 0.2) (layer "B.Cu") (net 3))
 (segment (start 156.36 90.84) (end 153.54 88.02) (width 0.2) (layer "B.Cu") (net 3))
 (segment (start 153.54 82.78) (end 153.39 82.63) (width 0.2) (layer "B.Cu") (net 3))
 (segment (start 153.54 88.02) (end 153.54 82.78) (width 0.2) (layer "B.Cu") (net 3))
 (segment (start 155.759 96.109) (end 150.73 91.08) (width 0.2) (layer "F.Cu") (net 9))
 (segment (start 162.22 104.19) (end 156.450057 104.19) (width 0.2) (layer "F.Cu") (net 9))
 (segment (start 155.759 103.498943) (end 155.759 96.109) (width 0.2) (layer "F.Cu") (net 9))
 (segment (start 146.840057 86.61) (end 145.889 85.658943) (width 0.2) (layer "F.Cu") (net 9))
 (segment (start 145.889 84.12575) (end 148.4045 81.61025) (width 0.2) (layer "F.Cu") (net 9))
 (segment (start 180.53 112.13) (end 178.441 110.041) (width 0.2) (layer "F.Cu") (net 9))
 (segment (start 175.309 110.041) (end 175.11 110.24) (width 0.2) (layer "F.Cu") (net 9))
 (segment (start 178.441 110.041) (end 175.309 110.041) (width 0.2) (layer "F.Cu") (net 9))
 (segment (start 156.450057 104.19) (end 155.759 103.498943) (width 0.2) (layer "F.Cu") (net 9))
 (segment (start 148.7 86.61) (end 146.840057 86.61) (width 0.2) (layer "F.Cu") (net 9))
 (segment (start 145.889 85.658943) (end 145.889 84.12575) (width 0.2) (layer "F.Cu") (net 9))
 (via (at 175.11 110.24) (size 0.6) (drill 0.3) (layers "F.Cu" "B.Cu") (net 9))
 (via (at 148.7 86.61) (size 0.6) (drill 0.3) (layers "F.Cu" "B.Cu") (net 9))
 (via (at 162.22 104.19) (size 0.6) (drill 0.3) (layers "F.Cu" "B.Cu") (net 9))
 (via (at 150.73 91.08) (size 0.6) (drill 0.3) (layers "F.Cu" "B.Cu") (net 9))
 (segment (start 150.73 88.64) (end 148.7 86.61) (width 0.2) (layer "B.Cu") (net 9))
 (segment (start 150.73 91.08) (end 150.73 88.64) (width 0.2) (layer "B.Cu") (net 9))
 (segment (start 175.11 110.24) (end 169.06 104.19) (width 0.2) (layer "B.Cu") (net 9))
 (segment (start 169.06 104.19) (end 162.22 104.19) (width 0.2) (layer "B.Cu") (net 9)))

